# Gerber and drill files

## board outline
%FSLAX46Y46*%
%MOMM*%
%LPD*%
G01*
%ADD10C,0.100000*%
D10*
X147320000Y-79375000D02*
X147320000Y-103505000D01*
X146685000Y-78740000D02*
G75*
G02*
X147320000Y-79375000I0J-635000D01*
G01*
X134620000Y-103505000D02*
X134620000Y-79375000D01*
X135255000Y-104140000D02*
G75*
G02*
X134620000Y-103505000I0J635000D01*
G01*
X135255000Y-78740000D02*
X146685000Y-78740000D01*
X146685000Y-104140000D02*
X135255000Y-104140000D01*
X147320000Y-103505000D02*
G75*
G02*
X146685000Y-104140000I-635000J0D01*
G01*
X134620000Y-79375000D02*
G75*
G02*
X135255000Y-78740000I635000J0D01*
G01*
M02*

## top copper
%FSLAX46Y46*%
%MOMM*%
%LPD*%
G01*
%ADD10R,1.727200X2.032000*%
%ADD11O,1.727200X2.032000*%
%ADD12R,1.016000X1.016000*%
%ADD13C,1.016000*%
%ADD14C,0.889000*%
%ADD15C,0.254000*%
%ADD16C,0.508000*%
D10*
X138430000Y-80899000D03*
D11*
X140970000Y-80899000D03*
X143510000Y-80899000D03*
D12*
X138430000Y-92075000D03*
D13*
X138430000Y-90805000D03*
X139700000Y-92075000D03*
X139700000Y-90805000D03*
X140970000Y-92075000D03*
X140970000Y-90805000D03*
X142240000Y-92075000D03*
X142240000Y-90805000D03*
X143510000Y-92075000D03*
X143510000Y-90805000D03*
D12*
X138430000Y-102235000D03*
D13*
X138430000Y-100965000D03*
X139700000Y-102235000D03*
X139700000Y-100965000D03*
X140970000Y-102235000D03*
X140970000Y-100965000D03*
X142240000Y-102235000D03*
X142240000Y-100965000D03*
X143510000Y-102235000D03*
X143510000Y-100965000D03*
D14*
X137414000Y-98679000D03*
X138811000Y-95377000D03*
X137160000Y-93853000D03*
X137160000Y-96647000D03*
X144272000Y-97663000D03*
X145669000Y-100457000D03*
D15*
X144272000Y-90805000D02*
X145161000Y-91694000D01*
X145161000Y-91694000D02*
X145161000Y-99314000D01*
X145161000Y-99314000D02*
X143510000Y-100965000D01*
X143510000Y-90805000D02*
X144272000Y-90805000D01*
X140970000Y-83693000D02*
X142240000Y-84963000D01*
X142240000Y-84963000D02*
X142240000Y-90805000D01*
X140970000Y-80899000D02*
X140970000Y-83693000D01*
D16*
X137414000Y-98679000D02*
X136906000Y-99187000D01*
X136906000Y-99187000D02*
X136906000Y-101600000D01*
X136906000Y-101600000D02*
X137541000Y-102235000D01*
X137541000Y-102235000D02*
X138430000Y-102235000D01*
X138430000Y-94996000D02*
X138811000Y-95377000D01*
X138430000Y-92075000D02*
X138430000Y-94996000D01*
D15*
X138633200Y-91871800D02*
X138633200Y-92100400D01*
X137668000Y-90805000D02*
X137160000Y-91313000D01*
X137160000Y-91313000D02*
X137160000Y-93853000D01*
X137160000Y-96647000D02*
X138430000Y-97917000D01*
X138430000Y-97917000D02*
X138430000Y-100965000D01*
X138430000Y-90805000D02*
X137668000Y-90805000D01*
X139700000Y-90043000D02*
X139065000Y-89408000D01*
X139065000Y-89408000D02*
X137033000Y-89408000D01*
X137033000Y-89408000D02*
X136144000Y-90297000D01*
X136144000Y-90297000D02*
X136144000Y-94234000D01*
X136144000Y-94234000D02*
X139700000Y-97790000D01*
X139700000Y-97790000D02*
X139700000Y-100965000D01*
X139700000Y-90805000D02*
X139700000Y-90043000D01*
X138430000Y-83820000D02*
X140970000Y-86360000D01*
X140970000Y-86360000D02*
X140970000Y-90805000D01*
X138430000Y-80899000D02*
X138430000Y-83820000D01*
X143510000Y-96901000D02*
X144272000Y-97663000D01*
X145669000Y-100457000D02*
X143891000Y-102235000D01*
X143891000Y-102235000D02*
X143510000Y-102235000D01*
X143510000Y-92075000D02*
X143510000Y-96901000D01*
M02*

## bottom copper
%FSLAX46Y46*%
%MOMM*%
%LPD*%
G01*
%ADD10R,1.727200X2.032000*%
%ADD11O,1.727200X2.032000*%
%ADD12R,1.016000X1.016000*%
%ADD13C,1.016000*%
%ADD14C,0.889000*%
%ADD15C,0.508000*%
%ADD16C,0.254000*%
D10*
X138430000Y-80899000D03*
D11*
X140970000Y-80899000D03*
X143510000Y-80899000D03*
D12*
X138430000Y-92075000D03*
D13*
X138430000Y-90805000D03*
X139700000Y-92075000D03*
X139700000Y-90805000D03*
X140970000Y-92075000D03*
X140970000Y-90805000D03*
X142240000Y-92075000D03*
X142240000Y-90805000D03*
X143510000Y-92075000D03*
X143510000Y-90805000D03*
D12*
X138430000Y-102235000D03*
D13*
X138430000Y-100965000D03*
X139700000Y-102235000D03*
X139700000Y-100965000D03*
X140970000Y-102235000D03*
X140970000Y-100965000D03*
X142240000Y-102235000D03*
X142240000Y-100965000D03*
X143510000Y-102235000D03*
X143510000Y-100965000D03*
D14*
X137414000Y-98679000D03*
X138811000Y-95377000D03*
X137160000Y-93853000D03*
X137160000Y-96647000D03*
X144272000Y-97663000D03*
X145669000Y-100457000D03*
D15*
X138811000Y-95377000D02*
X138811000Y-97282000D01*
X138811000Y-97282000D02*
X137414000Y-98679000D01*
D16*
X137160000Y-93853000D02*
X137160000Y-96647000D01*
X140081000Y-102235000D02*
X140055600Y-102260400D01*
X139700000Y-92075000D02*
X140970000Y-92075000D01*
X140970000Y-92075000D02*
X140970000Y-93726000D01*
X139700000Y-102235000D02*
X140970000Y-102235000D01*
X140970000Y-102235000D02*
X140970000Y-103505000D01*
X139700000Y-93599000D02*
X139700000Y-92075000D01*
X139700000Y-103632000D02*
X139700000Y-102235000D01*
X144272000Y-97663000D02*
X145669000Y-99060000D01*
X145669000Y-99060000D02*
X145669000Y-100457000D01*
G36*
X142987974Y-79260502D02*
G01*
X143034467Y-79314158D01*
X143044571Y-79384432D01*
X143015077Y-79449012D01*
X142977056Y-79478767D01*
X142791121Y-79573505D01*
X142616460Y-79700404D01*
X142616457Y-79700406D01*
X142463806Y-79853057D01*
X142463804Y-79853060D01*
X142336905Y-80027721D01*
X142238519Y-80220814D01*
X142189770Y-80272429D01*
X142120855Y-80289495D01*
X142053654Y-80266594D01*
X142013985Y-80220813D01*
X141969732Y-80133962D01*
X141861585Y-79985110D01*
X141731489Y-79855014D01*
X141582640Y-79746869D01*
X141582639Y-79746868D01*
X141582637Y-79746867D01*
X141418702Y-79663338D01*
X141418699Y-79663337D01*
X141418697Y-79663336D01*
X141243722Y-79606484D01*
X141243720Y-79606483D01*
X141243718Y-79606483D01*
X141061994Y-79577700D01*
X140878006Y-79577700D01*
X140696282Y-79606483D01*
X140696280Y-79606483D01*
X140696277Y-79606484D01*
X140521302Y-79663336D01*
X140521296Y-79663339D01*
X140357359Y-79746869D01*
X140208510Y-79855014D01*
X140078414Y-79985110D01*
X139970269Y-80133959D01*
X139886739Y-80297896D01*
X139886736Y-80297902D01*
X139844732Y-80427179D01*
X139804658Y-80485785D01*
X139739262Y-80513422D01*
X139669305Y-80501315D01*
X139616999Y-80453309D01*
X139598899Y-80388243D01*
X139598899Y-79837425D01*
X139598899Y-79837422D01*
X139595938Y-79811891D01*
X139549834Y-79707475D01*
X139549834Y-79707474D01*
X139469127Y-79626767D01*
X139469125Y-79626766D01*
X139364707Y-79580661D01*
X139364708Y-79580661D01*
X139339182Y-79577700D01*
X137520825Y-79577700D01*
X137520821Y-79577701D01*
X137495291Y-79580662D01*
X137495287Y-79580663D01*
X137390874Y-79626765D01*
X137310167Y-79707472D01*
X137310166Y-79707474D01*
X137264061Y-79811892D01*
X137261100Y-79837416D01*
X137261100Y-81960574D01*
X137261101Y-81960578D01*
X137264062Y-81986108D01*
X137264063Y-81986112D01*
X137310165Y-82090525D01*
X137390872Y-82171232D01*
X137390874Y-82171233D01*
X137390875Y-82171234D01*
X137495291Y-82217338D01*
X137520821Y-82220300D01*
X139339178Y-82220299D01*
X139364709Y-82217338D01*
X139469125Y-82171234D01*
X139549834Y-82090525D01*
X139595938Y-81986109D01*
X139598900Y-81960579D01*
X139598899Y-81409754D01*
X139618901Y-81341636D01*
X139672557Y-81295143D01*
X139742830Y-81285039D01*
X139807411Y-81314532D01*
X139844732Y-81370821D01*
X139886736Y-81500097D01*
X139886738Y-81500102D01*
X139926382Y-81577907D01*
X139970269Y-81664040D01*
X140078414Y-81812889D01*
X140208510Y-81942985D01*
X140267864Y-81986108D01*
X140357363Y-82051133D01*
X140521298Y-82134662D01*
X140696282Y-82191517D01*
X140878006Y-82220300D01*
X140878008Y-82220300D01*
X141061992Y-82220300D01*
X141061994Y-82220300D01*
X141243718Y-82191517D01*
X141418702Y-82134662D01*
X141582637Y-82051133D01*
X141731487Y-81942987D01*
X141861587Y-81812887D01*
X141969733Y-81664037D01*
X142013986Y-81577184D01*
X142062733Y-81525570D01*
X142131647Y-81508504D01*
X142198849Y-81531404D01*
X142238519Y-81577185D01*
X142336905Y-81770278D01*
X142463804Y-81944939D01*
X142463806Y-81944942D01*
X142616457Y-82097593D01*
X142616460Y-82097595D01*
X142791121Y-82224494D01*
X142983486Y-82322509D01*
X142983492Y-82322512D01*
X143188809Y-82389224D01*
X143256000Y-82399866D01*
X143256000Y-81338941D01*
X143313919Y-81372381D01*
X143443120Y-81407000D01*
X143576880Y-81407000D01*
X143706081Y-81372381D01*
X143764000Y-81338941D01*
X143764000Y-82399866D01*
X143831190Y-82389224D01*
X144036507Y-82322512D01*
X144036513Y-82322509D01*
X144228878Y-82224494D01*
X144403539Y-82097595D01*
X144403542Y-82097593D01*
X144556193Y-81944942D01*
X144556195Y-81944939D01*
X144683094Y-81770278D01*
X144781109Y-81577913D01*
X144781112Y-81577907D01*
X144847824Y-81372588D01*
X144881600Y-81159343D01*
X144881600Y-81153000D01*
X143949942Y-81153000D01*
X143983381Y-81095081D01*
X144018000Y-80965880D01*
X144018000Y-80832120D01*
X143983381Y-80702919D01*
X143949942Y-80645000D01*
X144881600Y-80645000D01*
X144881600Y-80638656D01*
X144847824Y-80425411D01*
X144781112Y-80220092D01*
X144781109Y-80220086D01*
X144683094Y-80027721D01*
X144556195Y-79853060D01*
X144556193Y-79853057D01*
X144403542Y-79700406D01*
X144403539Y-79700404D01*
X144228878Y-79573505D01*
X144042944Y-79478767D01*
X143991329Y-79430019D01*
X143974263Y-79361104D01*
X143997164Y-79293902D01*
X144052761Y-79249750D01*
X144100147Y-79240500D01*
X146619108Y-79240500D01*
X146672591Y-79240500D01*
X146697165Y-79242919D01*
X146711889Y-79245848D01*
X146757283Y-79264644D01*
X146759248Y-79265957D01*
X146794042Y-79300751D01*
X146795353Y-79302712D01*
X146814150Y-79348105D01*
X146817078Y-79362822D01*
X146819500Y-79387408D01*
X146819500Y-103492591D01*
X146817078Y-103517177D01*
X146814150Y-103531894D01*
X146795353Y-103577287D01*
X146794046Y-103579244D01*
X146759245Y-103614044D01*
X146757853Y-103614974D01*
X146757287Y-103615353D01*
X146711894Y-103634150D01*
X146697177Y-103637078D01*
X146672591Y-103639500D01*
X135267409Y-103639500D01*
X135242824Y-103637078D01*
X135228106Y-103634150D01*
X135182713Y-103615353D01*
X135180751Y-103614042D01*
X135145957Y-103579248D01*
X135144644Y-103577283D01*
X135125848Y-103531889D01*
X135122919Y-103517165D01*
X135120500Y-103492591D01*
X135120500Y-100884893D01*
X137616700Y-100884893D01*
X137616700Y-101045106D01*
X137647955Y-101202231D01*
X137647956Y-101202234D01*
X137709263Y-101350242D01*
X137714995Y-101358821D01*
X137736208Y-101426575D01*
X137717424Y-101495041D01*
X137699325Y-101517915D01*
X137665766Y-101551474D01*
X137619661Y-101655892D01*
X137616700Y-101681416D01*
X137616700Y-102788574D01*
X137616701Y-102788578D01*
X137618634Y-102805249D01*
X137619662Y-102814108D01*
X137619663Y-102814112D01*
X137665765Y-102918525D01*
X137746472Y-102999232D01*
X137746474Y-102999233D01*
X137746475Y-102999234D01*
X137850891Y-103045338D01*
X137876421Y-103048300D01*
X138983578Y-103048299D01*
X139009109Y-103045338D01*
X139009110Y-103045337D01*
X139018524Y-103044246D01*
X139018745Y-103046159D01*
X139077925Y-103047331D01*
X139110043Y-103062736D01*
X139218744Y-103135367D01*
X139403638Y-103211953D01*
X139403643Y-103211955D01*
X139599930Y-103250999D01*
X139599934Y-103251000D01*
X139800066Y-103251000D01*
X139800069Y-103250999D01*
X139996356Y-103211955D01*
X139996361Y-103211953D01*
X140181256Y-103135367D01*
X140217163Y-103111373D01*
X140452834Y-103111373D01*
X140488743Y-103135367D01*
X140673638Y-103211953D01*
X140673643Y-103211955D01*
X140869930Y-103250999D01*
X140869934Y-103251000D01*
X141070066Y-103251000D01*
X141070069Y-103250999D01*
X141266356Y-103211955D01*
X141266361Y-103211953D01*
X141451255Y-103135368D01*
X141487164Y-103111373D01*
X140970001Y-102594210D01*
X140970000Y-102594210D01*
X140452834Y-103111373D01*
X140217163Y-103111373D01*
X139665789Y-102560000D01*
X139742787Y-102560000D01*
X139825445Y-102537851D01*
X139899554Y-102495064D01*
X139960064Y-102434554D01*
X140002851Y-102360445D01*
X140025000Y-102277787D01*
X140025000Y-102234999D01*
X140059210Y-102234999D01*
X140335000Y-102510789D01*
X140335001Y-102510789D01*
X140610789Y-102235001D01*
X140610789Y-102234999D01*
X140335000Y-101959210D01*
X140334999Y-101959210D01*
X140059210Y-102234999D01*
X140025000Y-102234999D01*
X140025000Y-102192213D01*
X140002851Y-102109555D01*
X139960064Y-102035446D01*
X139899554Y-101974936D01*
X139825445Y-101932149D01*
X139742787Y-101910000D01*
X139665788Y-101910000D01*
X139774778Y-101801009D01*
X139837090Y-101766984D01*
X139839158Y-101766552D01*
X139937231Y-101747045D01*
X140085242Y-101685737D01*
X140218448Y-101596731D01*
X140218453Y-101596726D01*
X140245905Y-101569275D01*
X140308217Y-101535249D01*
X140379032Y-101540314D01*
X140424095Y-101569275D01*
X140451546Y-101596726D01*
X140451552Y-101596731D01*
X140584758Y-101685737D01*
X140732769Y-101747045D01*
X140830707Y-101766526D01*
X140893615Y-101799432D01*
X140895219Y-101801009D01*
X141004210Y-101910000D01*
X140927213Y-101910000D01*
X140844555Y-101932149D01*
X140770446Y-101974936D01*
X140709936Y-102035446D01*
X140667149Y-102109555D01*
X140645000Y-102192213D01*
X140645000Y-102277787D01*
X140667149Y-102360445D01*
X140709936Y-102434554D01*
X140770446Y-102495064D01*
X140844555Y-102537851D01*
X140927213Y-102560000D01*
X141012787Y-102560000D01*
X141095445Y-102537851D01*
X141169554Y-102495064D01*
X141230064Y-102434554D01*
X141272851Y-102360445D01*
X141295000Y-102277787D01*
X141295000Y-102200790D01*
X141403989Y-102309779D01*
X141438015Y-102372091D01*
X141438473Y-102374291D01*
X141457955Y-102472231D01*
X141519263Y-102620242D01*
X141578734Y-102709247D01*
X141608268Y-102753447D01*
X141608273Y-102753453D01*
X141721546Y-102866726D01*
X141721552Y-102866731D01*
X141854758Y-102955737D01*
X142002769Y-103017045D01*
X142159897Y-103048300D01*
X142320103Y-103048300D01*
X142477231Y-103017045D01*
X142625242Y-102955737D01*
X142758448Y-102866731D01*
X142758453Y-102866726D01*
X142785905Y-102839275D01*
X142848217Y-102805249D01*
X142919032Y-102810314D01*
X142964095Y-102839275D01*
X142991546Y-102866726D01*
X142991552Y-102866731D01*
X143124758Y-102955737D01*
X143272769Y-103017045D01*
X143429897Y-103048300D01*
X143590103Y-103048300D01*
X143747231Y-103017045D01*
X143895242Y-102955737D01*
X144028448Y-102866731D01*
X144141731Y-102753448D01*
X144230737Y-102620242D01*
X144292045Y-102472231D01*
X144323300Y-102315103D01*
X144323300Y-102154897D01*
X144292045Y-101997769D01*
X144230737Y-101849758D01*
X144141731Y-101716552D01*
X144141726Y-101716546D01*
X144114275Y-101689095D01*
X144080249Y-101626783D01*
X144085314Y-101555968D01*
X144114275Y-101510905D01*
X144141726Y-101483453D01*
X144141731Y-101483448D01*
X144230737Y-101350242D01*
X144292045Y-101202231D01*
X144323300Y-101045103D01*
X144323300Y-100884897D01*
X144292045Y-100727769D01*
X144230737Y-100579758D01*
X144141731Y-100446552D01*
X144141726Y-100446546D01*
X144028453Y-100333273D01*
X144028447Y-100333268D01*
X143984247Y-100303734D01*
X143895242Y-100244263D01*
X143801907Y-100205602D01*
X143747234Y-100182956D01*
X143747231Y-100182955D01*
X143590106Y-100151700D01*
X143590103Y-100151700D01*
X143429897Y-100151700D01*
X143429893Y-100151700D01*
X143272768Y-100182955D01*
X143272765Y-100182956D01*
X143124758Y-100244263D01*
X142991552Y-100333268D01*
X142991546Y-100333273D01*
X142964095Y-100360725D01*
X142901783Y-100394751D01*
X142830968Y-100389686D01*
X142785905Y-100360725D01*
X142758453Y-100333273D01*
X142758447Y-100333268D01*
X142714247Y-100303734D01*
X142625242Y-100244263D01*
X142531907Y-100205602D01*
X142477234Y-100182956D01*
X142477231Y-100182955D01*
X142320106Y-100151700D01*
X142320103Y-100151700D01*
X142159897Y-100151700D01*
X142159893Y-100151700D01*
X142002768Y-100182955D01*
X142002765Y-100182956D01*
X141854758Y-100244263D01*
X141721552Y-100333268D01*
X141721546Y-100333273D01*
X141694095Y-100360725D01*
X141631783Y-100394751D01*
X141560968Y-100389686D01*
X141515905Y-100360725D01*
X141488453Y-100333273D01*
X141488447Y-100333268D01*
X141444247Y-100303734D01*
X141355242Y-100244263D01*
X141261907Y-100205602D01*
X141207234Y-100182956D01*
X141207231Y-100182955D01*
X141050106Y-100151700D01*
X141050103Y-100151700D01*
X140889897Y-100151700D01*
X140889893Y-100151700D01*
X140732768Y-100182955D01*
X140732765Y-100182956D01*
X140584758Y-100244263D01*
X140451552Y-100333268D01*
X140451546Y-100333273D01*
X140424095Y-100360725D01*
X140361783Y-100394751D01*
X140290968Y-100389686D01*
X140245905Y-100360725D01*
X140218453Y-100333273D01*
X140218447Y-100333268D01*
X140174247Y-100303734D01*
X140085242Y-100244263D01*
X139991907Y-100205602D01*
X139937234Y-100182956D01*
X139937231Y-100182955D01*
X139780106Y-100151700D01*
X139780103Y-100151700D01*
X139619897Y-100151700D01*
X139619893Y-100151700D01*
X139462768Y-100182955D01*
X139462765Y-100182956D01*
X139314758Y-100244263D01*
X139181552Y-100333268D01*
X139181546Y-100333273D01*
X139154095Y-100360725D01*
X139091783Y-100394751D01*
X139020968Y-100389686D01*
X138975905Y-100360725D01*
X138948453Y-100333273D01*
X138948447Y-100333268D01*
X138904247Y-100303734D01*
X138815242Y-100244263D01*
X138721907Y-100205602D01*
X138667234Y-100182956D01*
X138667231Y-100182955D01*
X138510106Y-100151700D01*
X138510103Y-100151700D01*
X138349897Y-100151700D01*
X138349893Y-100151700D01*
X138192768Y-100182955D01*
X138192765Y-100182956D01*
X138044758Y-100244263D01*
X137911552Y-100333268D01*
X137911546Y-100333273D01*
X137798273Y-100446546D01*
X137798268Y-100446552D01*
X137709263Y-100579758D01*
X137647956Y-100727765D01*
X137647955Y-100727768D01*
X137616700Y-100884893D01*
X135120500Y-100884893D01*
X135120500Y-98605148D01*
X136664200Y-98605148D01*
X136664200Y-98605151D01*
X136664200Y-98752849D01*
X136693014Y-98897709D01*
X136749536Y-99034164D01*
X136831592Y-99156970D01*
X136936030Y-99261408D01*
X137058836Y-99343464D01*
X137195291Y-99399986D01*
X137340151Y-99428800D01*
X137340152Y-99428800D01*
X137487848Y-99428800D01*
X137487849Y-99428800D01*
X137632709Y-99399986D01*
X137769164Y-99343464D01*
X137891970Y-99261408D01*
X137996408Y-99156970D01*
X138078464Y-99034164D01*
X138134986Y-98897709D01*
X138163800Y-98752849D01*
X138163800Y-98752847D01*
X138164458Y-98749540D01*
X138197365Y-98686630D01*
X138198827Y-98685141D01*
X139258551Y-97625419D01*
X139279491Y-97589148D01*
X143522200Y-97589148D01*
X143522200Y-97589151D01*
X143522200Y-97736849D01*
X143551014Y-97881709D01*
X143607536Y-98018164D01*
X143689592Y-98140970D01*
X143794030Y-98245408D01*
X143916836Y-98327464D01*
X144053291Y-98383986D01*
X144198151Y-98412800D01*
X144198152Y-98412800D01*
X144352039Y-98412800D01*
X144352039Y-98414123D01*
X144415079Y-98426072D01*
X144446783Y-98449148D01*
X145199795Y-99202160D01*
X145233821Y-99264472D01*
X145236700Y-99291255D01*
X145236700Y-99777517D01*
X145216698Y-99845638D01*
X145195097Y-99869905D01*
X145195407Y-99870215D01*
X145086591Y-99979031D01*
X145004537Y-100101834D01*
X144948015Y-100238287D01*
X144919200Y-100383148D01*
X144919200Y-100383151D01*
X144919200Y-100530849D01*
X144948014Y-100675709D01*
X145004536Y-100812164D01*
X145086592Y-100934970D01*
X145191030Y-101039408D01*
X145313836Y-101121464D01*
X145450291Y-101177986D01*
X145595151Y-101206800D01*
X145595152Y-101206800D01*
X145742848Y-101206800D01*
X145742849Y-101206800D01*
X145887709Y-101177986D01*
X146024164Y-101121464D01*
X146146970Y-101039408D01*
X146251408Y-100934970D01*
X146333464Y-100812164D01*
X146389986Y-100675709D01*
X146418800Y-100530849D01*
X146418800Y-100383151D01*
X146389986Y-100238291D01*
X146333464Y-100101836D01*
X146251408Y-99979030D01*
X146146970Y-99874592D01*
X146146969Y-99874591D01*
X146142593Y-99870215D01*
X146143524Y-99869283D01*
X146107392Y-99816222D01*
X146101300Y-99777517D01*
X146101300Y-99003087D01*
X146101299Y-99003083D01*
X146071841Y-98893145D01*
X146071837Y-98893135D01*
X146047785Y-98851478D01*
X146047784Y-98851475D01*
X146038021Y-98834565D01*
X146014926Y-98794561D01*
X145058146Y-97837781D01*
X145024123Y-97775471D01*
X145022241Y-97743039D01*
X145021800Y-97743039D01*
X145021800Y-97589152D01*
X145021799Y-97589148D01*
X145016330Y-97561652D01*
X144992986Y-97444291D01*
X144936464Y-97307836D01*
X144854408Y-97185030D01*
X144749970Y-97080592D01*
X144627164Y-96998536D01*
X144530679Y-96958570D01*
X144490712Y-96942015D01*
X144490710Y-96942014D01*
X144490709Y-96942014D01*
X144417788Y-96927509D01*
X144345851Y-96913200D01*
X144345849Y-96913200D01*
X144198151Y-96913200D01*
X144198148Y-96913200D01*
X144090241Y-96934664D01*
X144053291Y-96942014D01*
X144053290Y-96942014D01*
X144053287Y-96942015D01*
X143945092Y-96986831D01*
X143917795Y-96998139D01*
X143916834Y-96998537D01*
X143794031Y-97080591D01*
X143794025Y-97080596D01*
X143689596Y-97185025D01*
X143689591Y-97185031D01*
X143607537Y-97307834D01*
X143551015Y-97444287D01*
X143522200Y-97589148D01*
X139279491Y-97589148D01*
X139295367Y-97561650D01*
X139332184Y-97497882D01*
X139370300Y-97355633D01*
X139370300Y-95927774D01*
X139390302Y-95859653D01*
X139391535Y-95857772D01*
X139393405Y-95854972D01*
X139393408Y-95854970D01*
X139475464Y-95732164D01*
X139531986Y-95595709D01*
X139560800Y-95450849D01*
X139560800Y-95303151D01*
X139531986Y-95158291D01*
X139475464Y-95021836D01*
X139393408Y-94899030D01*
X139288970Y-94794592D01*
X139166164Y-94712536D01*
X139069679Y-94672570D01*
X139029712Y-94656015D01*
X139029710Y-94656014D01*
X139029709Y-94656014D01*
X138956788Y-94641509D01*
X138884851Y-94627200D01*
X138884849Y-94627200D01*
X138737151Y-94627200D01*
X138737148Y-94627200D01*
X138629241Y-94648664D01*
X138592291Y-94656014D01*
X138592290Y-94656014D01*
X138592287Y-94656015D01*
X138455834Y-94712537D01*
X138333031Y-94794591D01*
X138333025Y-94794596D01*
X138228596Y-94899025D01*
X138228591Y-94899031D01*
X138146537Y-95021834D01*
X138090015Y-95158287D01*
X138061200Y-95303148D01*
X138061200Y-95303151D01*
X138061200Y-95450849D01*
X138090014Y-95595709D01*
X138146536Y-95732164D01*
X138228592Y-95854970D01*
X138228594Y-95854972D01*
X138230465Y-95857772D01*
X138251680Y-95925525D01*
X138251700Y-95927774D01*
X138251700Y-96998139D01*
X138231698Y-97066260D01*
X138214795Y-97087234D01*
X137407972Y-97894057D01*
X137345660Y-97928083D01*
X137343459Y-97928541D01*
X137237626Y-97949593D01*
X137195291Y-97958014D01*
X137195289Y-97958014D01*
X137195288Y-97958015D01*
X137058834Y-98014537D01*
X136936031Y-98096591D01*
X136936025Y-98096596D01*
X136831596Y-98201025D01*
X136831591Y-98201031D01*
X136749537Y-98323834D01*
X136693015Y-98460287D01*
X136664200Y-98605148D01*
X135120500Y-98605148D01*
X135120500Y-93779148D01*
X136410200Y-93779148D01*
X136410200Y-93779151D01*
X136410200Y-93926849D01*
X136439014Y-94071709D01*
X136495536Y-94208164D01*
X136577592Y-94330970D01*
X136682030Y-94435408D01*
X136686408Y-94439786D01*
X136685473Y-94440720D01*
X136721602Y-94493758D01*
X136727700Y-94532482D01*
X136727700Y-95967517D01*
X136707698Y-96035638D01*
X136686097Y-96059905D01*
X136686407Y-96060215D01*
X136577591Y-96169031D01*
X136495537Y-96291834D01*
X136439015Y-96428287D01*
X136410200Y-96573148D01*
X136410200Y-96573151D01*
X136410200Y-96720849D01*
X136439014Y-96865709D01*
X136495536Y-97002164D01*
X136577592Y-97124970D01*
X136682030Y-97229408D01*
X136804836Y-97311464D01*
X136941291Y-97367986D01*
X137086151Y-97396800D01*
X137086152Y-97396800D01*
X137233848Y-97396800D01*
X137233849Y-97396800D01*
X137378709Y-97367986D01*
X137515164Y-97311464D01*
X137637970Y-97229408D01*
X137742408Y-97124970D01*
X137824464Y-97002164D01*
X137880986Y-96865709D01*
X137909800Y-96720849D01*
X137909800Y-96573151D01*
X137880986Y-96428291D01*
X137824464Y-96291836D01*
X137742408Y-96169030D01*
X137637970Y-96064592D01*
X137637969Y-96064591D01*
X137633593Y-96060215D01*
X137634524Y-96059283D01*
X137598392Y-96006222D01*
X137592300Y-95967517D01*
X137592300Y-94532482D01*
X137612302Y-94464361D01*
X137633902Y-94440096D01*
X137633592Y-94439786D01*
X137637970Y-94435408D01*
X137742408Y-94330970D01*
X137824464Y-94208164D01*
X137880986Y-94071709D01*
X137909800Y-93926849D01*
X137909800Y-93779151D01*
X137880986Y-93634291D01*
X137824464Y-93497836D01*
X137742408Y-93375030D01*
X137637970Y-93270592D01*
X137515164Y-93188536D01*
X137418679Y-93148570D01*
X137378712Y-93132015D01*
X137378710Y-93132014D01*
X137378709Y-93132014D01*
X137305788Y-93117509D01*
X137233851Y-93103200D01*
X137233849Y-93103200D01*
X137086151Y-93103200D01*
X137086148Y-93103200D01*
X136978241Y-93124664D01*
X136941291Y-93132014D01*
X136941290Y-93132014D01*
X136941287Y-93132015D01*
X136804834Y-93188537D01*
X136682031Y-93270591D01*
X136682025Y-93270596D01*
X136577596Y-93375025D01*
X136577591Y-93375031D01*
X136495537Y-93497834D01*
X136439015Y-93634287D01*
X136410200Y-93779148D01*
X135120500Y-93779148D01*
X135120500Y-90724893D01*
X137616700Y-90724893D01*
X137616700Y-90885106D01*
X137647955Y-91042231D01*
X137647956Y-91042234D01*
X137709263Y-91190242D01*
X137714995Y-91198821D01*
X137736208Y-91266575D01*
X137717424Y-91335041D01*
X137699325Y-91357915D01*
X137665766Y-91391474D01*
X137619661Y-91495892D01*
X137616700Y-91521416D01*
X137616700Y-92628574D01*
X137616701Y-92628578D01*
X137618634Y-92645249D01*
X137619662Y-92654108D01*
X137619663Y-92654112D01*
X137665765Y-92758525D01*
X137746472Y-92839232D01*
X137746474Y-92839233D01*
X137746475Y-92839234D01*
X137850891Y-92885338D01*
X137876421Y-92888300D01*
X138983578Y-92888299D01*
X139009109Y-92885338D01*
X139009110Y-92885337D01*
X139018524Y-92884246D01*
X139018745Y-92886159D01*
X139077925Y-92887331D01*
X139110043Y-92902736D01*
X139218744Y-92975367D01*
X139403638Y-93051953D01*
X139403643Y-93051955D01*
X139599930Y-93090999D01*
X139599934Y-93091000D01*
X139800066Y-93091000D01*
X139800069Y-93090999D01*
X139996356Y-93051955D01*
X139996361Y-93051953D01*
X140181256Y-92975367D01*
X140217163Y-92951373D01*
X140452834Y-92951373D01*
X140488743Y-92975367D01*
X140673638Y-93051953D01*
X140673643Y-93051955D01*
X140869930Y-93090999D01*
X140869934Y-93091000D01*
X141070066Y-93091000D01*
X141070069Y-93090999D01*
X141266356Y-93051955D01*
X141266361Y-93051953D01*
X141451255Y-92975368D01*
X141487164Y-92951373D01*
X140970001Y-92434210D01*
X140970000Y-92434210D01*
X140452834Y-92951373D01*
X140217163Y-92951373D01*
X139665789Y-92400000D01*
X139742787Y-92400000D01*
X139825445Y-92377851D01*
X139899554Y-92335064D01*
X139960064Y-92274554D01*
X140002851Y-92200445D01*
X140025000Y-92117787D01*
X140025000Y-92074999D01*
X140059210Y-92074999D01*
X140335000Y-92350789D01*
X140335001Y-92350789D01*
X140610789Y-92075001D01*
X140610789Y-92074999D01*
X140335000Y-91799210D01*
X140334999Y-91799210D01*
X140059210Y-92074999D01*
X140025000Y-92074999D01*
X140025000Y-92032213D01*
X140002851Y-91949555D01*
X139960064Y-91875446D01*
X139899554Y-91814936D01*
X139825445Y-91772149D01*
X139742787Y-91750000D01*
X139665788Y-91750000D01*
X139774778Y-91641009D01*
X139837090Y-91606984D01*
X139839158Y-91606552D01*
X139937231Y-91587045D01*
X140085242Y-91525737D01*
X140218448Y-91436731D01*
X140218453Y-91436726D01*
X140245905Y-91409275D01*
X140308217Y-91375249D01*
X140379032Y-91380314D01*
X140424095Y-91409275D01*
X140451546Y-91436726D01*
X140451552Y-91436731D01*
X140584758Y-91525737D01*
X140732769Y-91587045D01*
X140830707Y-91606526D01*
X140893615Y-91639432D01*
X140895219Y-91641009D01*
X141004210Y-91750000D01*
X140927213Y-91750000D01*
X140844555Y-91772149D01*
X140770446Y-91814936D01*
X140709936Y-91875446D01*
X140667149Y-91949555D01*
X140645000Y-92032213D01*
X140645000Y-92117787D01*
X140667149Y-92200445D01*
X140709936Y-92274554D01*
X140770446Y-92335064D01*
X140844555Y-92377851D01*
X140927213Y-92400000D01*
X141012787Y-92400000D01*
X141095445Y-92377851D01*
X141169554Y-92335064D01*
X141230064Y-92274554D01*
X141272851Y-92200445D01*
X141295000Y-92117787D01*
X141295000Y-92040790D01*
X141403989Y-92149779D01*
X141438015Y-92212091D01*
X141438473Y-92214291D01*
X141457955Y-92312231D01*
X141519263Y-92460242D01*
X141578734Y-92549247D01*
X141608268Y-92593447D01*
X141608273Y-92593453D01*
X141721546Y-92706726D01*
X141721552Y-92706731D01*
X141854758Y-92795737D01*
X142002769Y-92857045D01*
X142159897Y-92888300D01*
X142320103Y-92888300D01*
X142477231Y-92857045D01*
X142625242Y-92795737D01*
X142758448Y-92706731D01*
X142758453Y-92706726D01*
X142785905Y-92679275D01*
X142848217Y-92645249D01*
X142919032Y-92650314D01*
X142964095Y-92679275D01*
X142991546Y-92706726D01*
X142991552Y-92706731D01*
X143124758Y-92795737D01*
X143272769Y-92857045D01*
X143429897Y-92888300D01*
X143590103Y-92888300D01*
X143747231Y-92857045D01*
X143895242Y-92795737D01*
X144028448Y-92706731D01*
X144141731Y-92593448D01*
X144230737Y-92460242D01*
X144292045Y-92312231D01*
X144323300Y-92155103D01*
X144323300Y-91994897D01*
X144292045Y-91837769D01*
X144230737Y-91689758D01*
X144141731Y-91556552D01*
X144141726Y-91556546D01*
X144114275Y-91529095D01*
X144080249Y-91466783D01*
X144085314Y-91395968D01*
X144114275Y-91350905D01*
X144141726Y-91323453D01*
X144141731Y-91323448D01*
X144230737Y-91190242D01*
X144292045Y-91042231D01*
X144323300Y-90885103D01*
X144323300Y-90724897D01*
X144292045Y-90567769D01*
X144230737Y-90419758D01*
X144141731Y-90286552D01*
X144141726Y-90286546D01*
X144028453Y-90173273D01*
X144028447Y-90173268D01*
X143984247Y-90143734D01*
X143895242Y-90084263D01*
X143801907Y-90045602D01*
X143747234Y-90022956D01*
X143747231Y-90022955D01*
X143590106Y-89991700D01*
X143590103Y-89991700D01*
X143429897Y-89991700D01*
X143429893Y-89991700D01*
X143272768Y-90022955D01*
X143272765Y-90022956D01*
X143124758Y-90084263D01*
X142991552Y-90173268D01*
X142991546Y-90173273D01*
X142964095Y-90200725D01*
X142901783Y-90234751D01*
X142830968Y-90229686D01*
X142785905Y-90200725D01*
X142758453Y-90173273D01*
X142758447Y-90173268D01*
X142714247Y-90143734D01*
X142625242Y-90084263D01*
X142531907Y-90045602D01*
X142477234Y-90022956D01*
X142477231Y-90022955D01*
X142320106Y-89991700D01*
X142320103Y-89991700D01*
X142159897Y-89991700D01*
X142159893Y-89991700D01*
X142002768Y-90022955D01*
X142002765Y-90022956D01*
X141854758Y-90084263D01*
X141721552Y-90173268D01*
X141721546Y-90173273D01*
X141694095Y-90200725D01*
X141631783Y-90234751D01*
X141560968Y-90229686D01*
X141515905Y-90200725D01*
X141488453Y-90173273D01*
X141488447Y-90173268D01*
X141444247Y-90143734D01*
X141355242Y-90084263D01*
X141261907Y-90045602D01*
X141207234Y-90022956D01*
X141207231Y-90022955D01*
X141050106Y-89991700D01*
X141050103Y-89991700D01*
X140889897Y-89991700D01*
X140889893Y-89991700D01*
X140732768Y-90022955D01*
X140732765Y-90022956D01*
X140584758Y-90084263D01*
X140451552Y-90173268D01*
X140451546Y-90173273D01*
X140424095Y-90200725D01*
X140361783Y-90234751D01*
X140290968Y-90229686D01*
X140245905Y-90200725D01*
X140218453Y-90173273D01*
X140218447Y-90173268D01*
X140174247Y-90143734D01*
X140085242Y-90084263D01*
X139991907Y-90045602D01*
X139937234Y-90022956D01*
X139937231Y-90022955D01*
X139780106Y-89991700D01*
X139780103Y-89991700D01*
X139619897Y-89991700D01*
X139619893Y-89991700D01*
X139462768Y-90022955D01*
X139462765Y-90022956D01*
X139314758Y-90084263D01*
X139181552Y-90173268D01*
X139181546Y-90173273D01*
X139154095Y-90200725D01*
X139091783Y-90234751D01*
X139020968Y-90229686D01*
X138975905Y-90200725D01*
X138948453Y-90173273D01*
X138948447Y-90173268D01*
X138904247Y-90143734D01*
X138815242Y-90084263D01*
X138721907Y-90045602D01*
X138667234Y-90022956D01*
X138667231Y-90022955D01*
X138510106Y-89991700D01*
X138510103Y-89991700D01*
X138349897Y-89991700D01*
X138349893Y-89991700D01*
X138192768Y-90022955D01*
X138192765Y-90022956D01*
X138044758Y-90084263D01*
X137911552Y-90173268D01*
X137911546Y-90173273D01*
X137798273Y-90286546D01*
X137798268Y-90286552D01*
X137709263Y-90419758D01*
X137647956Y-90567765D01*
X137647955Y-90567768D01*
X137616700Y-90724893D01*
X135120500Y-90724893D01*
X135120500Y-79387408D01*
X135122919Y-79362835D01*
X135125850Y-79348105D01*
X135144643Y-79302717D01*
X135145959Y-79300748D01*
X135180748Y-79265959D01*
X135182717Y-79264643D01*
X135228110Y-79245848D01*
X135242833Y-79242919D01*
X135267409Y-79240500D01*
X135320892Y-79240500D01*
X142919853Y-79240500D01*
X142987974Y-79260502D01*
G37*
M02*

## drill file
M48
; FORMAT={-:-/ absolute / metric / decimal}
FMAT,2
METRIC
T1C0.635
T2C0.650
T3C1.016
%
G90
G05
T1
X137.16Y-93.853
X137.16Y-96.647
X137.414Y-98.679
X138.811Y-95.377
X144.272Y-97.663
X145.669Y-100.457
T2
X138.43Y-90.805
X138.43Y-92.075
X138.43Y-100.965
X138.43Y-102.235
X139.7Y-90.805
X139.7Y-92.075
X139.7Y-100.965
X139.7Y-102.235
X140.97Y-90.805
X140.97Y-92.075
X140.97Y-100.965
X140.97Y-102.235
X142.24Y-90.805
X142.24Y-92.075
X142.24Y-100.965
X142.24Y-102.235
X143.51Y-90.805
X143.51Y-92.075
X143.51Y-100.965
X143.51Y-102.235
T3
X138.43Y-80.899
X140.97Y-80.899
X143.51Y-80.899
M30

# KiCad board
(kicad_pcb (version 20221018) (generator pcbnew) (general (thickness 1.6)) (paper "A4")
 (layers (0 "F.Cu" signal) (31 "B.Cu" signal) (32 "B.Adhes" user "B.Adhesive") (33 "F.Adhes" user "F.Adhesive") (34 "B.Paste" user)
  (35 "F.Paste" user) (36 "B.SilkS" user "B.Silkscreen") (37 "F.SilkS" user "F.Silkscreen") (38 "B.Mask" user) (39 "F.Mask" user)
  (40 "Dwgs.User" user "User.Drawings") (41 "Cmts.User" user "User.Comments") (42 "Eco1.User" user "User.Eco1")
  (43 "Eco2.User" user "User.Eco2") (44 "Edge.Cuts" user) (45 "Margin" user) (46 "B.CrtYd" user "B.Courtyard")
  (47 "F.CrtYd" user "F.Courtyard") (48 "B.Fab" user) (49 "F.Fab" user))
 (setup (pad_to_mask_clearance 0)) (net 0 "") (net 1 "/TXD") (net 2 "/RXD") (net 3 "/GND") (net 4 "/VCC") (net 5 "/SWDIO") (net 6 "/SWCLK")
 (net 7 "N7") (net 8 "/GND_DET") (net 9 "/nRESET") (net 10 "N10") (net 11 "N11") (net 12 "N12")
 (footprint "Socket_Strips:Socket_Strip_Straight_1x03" (layer "F.Cu") (at 140.97 80.899 180)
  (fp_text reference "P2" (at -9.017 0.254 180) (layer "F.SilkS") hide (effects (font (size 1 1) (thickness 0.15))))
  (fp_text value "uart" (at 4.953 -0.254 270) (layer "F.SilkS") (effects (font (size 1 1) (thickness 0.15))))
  (pad "1" thru_hole rect (at 2.54 0) (size 1.7272 2.032) (drill 1.016) (layers "*.Cu" "*.Mask" "F.SilkS") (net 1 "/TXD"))
  (pad "2" thru_hole oval (at 0 0) (size 1.7272 2.032) (drill 1.016) (layers "*.Cu" "*.Mask" "F.SilkS") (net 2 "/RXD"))
  (pad "3" thru_hole oval (at -2.54 0) (size 1.7272 2.032) (drill 1.016) (layers "*.Cu" "*.Mask" "F.SilkS") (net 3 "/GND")))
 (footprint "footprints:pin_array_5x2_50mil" (layer "F.Cu") (at 139.7 91.44)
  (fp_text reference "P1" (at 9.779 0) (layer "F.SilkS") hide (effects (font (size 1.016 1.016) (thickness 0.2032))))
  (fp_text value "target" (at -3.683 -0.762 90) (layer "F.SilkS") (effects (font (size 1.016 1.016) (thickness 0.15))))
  (pad "1" thru_hole rect (at -1.27 0.635) (size 1.016 1.016) (drill 0.65) (layers "*.Cu" "*.Mask" "F.SilkS") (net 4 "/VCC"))
  (pad "2" thru_hole circle (at -1.27 -0.635) (size 1.016 1.016) (drill 0.65) (layers "*.Cu" "*.Mask" "F.SilkS") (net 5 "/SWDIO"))
  (pad "3" thru_hole circle (at 0 0.635) (size 1.016 1.016) (drill 0.65) (layers "*.Cu" "*.Mask" "F.SilkS") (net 3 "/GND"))
  (pad "4" thru_hole circle (at 0 -0.635) (size 1.016 1.016) (drill 0.65) (layers "*.Cu" "*.Mask" "F.SilkS") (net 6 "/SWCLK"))
  (pad "5" thru_hole circle (at 1.27 0.635) (size 1.016 1.016) (drill 0.65) (layers "*.Cu" "*.Mask" "F.SilkS") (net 3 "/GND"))
  (pad "6" thru_hole circle (at 1.27 -0.635) (size 1.016 1.016) (drill 0.65) (layers "*.Cu" "*.Mask" "F.SilkS") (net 1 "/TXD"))
  (pad "7" thru_hole circle (at 2.54 0.635) (size 1.016 1.016) (drill 0.65) (layers "*.Cu" "*.Mask" "F.SilkS") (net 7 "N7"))
  (pad "8" thru_hole circle (at 2.54 -0.635) (size 1.016 1.016) (drill 0.65) (layers "*.Cu" "*.Mask" "F.SilkS") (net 2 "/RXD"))
  (pad "9" thru_hole circle (at 3.81 0.635) (size 1.016 1.016) (drill 0.65) (layers "*.Cu" "*.Mask" "F.SilkS") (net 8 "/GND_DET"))
  (pad "10" thru_hole circle (at 3.81 -0.635) (size 1.016 1.016) (drill 0.65) (layers "*.Cu" "*.Mask" "F.SilkS") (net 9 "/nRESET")))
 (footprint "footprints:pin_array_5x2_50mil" (layer "F.Cu") (at 139.7 101.6)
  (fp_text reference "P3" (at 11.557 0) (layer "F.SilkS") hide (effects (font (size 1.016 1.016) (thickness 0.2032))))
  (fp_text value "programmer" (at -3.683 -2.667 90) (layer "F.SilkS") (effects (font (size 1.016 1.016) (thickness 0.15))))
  (pad "1" thru_hole rect (at -1.27 0.635) (size 1.016 1.016) (drill 0.65) (layers "*.Cu" "*.Mask" "F.SilkS") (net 4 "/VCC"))
  (pad "2" thru_hole circle (at -1.27 -0.635) (size 1.016 1.016) (drill 0.65) (layers "*.Cu" "*.Mask" "F.SilkS") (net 5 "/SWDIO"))
  (pad "3" thru_hole circle (at 0 0.635) (size 1.016 1.016) (drill 0.65) (layers "*.Cu" "*.Mask" "F.SilkS") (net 3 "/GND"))
  (pad "4" thru_hole circle (at 0 -0.635) (size 1.016 1.016) (drill 0.65) (layers "*.Cu" "*.Mask" "F.SilkS") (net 6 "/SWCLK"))
  (pad "5" thru_hole circle (at 1.27 0.635) (size 1.016 1.016) (drill 0.65) (layers "*.Cu" "*.Mask" "F.SilkS") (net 3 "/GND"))
  (pad "6" thru_hole circle (at 1.27 -0.635) (size 1.016 1.016) (drill 0.65) (layers "*.Cu" "*.Mask" "F.SilkS") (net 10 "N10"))
  (pad "7" thru_hole circle (at 2.54 0.635) (size 1.016 1.016) (drill 0.65) (layers "*.Cu" "*.Mask" "F.SilkS") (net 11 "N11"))
  (pad "8" thru_hole circle (at 2.54 -0.635) (size 1.016 1.016) (drill 0.65) (layers "*.Cu" "*.Mask" "F.SilkS") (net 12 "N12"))
  (pad "9" thru_hole circle (at 3.81 0.635) (size 1.016 1.016) (drill 0.65) (layers "*.Cu" "*.Mask" "F.SilkS") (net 8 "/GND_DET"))
  (pad "10" thru_hole circle (at 3.81 -0.635) (size 1.016 1.016) (drill 0.65) (layers "*.Cu" "*.Mask" "F.SilkS") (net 9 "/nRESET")))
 (gr_line (start 147.32 79.375) (end 147.32 103.505) (stroke (width 0.1) (type solid)) (layer "Edge.Cuts"))
 (gr_arc (start 146.685 78.74) (mid 147.134013 78.925987) (end 147.32 79.375) (stroke (width 0.1) (type solid)) (layer "Edge.Cuts"))
 (gr_line (start 134.62 103.505) (end 134.62 79.375) (stroke (width 0.1) (type solid)) (layer "Edge.Cuts"))
 (gr_arc (start 135.255 104.14) (mid 134.805987 103.954013) (end 134.62 103.505) (stroke (width 0.1) (type solid)) (layer "Edge.Cuts"))
 (gr_line (start 135.255 78.74) (end 146.685 78.74) (stroke (width 0.1) (type solid)) (layer "Edge.Cuts"))
 (gr_line (start 146.685 104.14) (end 135.255 104.14) (stroke (width 0.1) (type solid)) (layer "Edge.Cuts"))
 (gr_arc (start 147.32 103.505) (mid 147.134013 103.954013) (end 146.685 104.14) (stroke (width 0.1) (type solid)) (layer "Edge.Cuts"))
 (gr_arc (start 134.62 79.375) (mid 134.805987 78.925987) (end 135.255 78.74) (stroke (width 0.1) (type solid)) (layer "Edge.Cuts"))
 (segment (start 144.272 90.805) (end 145.161 91.694) (width 0.254) (layer "F.Cu") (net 9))
 (segment (start 145.161 91.694) (end 145.161 99.314) (width 0.254) (layer "F.Cu") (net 9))
 (segment (start 145.161 99.314) (end 143.51 100.965) (width 0.254) (layer "F.Cu") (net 9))
 (segment (start 143.51 90.805) (end 144.272 90.805) (width 0.254) (layer "F.Cu") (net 9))
 (segment (start 140.97 83.693) (end 142.24 84.963) (width 0.254) (layer "F.Cu") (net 2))
 (segment (start 142.24 84.963) (end 142.24 90.805) (width 0.254) (layer "F.Cu") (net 2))
 (segment (start 140.97 80.899) (end 140.97 83.693) (width 0.254) (layer "F.Cu") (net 2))
 (segment (start 137.414 98.679) (end 136.906 99.187) (width 0.508) (layer "F.Cu") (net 4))
 (segment (start 136.906 99.187) (end 136.906 101.6) (width 0.508) (layer "F.Cu") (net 4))
 (segment (start 136.906 101.6) (end 137.541 102.235) (width 0.508) (layer "F.Cu") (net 4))
 (segment (start 137.541 102.235) (end 138.43 102.235) (width 0.508) (layer "F.Cu") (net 4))
 (segment (start 138.43 94.996) (end 138.811 95.377) (width 0.508) (layer "F.Cu") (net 4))
 (segment (start 138.43 92.075) (end 138.43 94.996) (width 0.508) (layer "F.Cu") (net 4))
 (segment (start 138.6332 91.8718) (end 138.6332 92.1004) (width 0.254) (layer "F.Cu") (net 4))
 (via (at 137.414 98.679) (size 0.889) (drill 0.635) (layers "F.Cu" "B.Cu") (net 4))
 (via (at 138.811 95.377) (size 0.889) (drill 0.635) (layers "F.Cu" "B.Cu") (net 4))
 (segment (start 138.811 95.377) (end 138.811 97.282) (width 0.508) (layer "B.Cu") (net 4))
 (segment (start 138.811 97.282) (end 137.414 98.679) (width 0.508) (layer "B.Cu") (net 4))
 (segment (start 137.668 90.805) (end 137.16 91.313) (width 0.254) (layer "F.Cu") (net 5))
 (segment (start 137.16 91.313) (end 137.16 93.853) (width 0.254) (layer "F.Cu") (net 5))
 (segment (start 137.16 96.647) (end 138.43 97.917) (width 0.254) (layer "F.Cu") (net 5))
 (segment (start 138.43 97.917) (end 138.43 100.965) (width 0.254) (layer "F.Cu") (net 5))
 (segment (start 138.43 90.805) (end 137.668 90.805) (width 0.254) (layer "F.Cu") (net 5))
 (via (at 137.16 93.853) (size 0.889) (drill 0.635) (layers "F.Cu" "B.Cu") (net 5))
 (via (at 137.16 96.647) (size 0.889) (drill 0.635) (layers "F.Cu" "B.Cu") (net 5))
 (segment (start 137.16 93.853) (end 137.16 96.647) (width 0.254) (layer "B.Cu") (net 5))
 (segment (start 140.081 102.235) (end 140.0556 102.2604) (width 0.254) (layer "B.Cu") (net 3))
 (segment (start 139.7 92.075) (end 140.97 92.075) (width 0.254) (layer "B.Cu") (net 3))
 (segment (start 140.97 92.075) (end 140.97 93.726) (width 0.254) (layer "B.Cu") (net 3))
 (segment (start 139.7 102.235) (end 140.97 102.235) (width 0.254) (layer "B.Cu") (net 3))
 (segment (start 140.97 102.235) (end 140.97 103.505) (width 0.254) (layer "B.Cu") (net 3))
 (segment (start 139.7 93.599) (end 139.7 92.075) (width 0.254) (layer "B.Cu") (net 3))
 (segment (start 139.7 103.632) (end 139.7 102.235) (width 0.254) (layer "B.Cu") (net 3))
 (segment (start 139.7 90.043) (end 139.065 89.408) (width 0.254) (layer "F.Cu") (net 6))
 (segment (start 139.065 89.408) (end 137.033 89.408) (width 0.254) (layer "F.Cu") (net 6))
 (segment (start 137.033 89.408) (end 136.144 90.297) (width 0.254) (layer "F.Cu") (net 6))
 (segment (start 136.144 90.297) (end 136.144 94.234) (width 0.254) (layer "F.Cu") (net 6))
 (segment (start 136.144 94.234) (end 139.7 97.79) (width 0.254) (layer "F.Cu") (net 6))
 (segment (start 139.7 97.79) (end 139.7 100.965) (width 0.254) (layer "F.Cu") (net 6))
 (segment (start 139.7 90.805) (end 139.7 90.043) (width 0.254) (layer "F.Cu") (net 6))
 (segment (start 138.43 83.82) (end 140.97 86.36) (width 0.254) (layer "F.Cu") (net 1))
 (segment (start 140.97 86.36) (end 140.97 90.805) (width 0.254) (layer "F.Cu") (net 1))
 (segment (start 138.43 80.899) (end 138.43 83.82) (width 0.254) (layer "F.Cu") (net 1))
 (segment (start 143.51 96.901) (end 144.272 97.663) (width 0.254) (layer "F.Cu") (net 8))
 (segment (start 145.669 100.457) (end 143.891 102.235) (width 0.254) (layer "F.Cu") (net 8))
 (segment (start 143.891 102.235) (end 143.51 102.235) (width 0.254) (layer "F.Cu") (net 8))
 (segment (start 143.51 92.075) (end 143.51 96.901) (width 0.254) (layer "F.Cu") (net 8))
 (via (at 144.272 97.663) (size 0.889) (drill 0.635) (layers "F.Cu" "B.Cu") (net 8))
 (via (at 145.669 100.457) (size 0.889) (drill 0.635) (layers "F.Cu" "B.Cu") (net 8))
 (segment (start 144.272 97.663) (end 145.669 99.06) (width 0.254) (layer "B.Cu") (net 8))
 (segment (start 145.669 99.06) (end 145.669 100.457) (width 0.254) (layer "B.Cu") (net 8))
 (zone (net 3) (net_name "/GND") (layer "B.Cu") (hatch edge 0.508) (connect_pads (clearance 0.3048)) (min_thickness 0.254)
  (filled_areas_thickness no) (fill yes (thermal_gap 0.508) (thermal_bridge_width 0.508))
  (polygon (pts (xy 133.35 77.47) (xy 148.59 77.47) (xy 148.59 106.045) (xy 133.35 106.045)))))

